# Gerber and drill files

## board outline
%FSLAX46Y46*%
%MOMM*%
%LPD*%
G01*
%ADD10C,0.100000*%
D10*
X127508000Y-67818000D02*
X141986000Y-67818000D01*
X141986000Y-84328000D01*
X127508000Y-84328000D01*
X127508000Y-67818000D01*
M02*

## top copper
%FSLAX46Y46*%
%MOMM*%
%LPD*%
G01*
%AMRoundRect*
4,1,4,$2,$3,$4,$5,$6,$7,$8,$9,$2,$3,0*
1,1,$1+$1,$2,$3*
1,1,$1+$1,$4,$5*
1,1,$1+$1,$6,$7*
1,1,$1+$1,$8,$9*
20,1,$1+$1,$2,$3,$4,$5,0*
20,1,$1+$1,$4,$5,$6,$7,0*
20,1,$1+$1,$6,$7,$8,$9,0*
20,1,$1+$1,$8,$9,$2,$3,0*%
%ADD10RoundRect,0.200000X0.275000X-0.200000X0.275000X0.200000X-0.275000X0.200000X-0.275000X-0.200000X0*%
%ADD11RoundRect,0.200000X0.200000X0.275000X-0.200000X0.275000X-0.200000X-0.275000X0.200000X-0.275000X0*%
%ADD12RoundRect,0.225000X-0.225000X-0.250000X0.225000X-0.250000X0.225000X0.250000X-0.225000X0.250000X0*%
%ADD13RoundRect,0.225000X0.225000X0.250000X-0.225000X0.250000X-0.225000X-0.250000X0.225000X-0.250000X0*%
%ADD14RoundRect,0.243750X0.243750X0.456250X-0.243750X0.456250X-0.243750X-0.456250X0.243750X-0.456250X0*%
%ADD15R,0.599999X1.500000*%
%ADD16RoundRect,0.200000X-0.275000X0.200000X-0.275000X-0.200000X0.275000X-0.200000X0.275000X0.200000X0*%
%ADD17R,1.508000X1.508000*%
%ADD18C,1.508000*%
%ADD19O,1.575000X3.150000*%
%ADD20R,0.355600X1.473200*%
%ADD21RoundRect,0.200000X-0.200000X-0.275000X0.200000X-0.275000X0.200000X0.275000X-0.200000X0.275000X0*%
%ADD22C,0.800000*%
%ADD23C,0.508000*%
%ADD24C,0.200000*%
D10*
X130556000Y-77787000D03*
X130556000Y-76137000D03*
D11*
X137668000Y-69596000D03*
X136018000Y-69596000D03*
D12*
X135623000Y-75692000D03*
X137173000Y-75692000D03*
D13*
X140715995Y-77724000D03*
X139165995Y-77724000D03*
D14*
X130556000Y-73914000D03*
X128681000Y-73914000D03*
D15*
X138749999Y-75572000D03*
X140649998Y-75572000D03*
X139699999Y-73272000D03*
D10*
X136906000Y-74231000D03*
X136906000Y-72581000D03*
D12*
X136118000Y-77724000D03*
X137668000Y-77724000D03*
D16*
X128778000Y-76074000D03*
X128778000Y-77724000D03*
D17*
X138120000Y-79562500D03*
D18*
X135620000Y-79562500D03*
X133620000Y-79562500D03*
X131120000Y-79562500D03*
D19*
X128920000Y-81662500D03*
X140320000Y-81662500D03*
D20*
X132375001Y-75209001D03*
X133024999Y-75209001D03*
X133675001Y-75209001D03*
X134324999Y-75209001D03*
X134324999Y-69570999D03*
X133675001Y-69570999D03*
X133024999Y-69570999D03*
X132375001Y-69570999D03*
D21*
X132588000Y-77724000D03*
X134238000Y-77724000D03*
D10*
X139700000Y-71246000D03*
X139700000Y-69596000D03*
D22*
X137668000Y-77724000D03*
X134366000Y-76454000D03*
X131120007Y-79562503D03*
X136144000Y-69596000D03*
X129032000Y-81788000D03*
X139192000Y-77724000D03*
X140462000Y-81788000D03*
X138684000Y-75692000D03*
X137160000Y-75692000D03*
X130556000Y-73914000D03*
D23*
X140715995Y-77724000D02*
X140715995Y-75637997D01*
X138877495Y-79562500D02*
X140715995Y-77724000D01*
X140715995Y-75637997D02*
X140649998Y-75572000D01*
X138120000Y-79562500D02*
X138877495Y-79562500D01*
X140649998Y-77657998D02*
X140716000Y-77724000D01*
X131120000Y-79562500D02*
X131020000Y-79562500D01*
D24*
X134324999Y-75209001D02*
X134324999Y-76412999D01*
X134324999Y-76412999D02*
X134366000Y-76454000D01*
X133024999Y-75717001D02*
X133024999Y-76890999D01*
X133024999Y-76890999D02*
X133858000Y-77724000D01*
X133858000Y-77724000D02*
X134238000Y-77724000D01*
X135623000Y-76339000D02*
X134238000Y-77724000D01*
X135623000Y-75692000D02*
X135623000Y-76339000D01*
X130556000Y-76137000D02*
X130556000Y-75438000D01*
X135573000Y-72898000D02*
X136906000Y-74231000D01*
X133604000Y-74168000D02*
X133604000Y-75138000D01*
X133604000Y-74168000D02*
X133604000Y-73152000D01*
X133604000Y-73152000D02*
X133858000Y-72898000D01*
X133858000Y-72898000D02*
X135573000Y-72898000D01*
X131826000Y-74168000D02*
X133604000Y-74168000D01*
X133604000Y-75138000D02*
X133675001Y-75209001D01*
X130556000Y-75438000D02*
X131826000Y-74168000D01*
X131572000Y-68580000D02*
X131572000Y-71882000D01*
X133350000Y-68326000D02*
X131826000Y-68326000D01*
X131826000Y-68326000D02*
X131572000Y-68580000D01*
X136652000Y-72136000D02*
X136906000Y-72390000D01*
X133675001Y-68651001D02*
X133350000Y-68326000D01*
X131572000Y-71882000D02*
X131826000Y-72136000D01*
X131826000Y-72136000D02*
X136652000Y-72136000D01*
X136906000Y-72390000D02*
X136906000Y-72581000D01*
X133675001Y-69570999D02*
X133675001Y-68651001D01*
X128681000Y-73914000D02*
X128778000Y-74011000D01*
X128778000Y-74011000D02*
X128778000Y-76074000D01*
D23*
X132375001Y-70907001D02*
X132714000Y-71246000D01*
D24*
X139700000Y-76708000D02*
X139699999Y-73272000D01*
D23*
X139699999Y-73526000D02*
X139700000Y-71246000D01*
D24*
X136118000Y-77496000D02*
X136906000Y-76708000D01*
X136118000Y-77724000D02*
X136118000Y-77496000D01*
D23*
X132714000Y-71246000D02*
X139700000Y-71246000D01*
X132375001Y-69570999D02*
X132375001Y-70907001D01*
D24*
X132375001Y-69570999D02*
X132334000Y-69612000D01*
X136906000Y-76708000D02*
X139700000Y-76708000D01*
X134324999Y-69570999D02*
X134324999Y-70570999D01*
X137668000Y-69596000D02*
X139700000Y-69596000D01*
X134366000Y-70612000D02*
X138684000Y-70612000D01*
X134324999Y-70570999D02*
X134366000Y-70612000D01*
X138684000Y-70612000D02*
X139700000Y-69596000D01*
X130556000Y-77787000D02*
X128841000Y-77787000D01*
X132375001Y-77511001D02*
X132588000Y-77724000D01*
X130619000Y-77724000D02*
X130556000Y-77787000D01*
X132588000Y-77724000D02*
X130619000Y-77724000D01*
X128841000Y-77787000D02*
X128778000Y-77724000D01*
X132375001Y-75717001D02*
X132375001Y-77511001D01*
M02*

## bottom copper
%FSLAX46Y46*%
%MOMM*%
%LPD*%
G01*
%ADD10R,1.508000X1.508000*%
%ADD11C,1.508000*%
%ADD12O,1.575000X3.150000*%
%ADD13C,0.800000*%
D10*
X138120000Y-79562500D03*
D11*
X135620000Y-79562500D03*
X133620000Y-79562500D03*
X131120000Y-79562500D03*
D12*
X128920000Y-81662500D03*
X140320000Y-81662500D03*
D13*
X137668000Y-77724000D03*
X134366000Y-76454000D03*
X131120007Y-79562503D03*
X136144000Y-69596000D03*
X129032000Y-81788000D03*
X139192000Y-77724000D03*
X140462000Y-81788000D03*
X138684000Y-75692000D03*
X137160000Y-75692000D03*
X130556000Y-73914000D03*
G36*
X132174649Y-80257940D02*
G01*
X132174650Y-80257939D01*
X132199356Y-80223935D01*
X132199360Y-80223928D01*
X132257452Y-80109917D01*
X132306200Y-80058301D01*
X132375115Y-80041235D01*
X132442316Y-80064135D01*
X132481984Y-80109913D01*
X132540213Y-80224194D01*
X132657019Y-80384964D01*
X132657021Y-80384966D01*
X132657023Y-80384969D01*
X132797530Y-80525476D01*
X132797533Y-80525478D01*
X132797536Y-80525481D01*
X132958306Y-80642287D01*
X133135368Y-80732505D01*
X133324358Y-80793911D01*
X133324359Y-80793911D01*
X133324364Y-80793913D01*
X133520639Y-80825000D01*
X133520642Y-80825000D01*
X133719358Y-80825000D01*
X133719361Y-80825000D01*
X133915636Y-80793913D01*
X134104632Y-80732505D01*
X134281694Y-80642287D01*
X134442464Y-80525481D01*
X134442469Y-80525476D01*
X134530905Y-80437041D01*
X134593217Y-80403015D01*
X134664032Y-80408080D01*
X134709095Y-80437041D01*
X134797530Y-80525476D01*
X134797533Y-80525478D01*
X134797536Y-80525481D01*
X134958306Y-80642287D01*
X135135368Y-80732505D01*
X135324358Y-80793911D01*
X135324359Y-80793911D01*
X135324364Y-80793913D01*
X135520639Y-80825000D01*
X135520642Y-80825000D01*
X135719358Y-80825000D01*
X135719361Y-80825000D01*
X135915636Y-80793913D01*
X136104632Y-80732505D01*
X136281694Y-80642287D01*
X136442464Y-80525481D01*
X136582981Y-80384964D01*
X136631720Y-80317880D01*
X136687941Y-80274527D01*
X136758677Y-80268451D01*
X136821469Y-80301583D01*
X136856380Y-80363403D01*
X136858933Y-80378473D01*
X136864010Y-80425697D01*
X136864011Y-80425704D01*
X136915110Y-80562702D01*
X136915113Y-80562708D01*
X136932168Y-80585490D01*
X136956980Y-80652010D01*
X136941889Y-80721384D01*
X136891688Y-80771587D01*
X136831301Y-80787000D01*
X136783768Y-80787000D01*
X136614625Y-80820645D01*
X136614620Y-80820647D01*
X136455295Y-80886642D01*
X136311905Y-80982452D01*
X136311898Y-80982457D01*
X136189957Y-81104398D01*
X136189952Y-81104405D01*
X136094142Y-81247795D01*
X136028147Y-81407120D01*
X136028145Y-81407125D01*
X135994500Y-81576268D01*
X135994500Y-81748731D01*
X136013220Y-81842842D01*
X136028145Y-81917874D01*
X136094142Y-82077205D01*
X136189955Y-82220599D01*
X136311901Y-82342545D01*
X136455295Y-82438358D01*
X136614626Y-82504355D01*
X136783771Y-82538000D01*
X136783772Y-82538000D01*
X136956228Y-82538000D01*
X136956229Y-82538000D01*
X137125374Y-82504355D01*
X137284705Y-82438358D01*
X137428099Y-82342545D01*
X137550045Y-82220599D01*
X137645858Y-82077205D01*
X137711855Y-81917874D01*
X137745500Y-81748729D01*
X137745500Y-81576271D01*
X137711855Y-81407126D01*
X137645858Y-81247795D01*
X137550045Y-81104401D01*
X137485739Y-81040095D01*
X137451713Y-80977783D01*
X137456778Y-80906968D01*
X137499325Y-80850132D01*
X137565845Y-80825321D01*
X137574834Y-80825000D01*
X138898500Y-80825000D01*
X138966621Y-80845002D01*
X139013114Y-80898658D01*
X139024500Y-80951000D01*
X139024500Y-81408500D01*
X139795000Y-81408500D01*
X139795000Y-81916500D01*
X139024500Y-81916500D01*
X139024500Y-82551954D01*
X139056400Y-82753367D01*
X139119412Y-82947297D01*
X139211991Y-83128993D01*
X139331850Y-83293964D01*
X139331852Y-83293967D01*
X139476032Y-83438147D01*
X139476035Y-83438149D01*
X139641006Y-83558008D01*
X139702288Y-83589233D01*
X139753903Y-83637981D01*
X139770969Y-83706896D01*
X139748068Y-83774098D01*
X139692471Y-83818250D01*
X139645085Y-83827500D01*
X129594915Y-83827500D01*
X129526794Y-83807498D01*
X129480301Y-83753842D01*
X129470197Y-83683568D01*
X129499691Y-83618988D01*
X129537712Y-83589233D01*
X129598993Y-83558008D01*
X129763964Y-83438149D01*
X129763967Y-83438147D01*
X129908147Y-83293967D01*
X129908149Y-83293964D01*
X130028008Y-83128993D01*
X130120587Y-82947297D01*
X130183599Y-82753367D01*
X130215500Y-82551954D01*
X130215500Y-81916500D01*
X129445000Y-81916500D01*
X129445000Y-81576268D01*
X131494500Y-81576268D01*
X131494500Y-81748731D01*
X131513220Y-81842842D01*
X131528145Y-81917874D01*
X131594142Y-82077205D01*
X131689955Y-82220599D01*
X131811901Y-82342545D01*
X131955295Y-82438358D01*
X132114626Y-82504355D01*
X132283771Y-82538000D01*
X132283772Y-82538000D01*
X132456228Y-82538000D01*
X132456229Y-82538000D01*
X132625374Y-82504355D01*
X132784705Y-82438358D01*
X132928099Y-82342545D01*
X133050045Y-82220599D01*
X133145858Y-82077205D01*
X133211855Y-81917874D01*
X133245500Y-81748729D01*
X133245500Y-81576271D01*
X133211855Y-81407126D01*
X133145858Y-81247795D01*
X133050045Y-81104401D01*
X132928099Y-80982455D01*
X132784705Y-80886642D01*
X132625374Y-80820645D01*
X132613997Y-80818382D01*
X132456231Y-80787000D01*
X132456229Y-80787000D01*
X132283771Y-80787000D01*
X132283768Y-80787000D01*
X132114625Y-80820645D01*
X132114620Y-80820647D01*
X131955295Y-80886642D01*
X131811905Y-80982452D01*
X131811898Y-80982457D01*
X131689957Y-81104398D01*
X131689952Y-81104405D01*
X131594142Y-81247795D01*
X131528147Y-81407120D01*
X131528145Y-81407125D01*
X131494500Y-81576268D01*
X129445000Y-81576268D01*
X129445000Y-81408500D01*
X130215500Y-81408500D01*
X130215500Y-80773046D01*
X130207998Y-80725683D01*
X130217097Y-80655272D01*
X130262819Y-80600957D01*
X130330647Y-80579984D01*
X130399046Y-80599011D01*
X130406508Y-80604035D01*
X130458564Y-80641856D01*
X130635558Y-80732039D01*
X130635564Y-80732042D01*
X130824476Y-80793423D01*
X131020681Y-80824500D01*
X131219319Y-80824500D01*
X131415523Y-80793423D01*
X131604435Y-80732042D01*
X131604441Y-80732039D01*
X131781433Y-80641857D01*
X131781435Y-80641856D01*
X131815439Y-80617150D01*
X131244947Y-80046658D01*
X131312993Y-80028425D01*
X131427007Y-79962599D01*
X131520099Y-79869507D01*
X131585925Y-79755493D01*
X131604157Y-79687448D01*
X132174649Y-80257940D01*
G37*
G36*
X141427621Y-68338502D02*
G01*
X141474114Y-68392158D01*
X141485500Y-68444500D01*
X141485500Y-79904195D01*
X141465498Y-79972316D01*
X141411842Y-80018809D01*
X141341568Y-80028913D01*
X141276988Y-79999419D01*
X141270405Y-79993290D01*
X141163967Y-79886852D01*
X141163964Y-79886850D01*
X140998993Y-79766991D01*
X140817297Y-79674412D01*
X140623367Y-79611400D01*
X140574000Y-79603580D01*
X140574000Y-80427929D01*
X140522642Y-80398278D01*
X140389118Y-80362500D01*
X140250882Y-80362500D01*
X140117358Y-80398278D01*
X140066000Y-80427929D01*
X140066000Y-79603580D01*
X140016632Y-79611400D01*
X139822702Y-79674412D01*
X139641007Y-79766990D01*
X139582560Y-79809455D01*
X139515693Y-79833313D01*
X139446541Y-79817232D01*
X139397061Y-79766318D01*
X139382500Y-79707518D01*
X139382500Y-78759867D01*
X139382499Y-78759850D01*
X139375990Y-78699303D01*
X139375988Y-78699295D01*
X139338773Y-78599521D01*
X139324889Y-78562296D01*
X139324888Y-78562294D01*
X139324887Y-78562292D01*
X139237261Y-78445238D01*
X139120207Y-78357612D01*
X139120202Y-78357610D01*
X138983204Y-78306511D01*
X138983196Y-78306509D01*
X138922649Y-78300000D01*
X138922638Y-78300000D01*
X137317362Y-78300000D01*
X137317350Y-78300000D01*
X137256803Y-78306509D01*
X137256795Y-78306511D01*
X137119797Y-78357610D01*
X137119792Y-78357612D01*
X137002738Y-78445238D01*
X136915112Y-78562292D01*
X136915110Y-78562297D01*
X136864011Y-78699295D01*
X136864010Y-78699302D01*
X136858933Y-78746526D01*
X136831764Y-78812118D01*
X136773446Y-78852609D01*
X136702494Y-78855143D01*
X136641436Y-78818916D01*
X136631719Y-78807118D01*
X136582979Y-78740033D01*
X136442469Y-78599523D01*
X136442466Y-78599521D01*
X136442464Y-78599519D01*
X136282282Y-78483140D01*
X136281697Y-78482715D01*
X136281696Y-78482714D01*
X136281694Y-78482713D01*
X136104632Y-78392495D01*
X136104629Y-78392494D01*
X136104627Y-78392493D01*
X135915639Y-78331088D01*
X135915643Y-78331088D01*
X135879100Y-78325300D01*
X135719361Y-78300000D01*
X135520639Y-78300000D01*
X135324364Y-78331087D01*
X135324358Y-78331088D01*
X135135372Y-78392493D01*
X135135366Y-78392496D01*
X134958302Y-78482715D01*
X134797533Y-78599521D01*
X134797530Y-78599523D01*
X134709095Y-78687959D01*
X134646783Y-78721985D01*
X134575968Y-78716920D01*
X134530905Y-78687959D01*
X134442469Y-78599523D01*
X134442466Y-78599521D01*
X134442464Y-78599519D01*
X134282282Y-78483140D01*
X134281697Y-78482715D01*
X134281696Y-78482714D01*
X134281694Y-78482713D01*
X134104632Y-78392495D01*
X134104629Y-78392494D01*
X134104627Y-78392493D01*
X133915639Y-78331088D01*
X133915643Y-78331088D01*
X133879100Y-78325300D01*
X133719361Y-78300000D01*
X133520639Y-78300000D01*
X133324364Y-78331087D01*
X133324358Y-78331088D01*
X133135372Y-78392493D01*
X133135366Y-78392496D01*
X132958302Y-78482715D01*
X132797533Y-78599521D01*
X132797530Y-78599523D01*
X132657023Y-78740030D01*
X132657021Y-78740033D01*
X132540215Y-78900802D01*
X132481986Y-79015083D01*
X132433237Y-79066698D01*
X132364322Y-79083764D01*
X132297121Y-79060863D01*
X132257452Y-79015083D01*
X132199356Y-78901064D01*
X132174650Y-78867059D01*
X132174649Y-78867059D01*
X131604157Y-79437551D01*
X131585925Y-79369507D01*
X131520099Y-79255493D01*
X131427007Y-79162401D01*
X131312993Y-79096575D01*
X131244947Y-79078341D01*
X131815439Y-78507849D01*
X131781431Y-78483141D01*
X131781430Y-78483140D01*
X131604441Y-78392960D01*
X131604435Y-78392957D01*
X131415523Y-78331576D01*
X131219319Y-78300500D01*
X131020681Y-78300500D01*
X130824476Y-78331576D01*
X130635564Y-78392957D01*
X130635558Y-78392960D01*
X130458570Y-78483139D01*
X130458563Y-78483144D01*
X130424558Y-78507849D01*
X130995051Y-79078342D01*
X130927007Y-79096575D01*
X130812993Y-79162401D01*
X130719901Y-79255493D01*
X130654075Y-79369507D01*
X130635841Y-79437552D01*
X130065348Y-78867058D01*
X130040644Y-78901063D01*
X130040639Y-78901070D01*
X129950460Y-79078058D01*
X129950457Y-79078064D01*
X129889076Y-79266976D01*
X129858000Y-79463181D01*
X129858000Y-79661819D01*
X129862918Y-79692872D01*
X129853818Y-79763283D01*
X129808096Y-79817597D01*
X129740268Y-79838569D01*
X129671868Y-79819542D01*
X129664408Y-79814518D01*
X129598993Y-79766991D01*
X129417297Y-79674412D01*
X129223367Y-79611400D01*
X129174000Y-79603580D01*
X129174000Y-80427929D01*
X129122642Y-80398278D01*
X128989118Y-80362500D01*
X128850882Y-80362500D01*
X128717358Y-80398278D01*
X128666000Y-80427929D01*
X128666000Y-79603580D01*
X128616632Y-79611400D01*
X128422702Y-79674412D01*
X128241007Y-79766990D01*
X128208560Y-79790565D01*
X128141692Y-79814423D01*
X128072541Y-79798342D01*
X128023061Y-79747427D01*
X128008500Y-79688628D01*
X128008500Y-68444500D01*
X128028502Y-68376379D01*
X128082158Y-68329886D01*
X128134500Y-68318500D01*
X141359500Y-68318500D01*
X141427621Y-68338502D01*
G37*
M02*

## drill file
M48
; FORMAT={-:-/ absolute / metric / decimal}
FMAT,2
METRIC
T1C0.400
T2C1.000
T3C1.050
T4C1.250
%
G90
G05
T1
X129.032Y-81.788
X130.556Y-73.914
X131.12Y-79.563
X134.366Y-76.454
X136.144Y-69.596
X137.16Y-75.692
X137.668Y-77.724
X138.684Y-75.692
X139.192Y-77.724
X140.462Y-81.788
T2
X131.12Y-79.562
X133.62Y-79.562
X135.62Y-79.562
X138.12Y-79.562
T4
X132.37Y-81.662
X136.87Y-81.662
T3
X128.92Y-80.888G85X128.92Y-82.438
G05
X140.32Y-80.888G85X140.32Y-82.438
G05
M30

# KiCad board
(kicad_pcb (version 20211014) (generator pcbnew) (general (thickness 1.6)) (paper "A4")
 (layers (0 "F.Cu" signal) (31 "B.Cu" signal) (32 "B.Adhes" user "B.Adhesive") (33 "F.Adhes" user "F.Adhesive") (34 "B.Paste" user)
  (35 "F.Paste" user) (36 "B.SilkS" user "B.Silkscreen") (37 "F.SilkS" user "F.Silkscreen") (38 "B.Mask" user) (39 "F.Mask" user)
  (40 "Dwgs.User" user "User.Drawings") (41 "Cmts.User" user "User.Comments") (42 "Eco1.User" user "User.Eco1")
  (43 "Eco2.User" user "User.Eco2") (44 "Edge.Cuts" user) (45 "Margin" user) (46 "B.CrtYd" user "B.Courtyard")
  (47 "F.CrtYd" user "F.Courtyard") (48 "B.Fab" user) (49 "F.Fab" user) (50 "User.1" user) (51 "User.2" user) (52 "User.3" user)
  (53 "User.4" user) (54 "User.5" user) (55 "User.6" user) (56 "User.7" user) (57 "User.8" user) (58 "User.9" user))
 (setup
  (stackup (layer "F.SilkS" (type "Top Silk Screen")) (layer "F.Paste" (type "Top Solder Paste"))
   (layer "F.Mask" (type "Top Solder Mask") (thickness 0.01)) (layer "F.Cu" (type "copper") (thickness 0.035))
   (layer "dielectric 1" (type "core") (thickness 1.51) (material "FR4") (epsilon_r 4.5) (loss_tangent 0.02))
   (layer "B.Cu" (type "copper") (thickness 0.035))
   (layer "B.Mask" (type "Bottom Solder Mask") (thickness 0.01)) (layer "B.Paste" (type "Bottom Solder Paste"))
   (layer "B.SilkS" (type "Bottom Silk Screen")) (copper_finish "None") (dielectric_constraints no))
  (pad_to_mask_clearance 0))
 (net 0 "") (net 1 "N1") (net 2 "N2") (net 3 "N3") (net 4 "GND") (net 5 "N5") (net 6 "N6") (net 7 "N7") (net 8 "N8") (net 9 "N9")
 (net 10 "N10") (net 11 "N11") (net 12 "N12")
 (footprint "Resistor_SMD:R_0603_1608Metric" (layer "F.Cu") (at 130.556 76.962 90)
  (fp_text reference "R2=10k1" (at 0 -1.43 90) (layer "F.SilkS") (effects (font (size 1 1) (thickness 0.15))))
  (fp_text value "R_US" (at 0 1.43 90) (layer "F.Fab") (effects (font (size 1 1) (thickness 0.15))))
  (pad "1" smd roundrect (at -0.825 0 90) (size 0.8 0.95) (layers "F.Cu" "F.Paste" "F.Mask") (roundrect_rratio 0.25) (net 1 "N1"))
  (pad "2" smd roundrect (at 0.825 0 90) (size 0.8 0.95) (layers "F.Cu" "F.Paste" "F.Mask") (roundrect_rratio 0.25) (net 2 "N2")))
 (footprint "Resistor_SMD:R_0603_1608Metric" (layer "F.Cu") (at 136.843 69.596 180)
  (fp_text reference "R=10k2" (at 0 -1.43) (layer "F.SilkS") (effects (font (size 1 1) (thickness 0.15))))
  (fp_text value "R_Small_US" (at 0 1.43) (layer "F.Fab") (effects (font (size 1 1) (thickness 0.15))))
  (pad "1" smd roundrect (at -0.825 0 180) (size 0.8 0.95) (layers "F.Cu" "F.Paste" "F.Mask") (roundrect_rratio 0.25) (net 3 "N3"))
  (pad "2" smd roundrect (at 0.825 0 180) (size 0.8 0.95) (layers "F.Cu" "F.Paste" "F.Mask") (roundrect_rratio 0.25) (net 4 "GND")))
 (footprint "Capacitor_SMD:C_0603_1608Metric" (layer "F.Cu") (at 136.398 75.692)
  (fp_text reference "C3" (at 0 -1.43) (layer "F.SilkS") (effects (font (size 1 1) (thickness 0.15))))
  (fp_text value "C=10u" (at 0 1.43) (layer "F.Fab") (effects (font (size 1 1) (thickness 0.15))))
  (pad "1" smd roundrect (at -0.775 0) (size 0.9 0.95) (layers "F.Cu" "F.Paste" "F.Mask") (roundrect_rratio 0.25) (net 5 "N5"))
  (pad "2" smd roundrect (at 0.775 0) (size 0.9 0.95) (layers "F.Cu" "F.Paste" "F.Mask") (roundrect_rratio 0.25) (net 4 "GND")))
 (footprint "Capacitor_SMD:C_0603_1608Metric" (layer "F.Cu") (at 139.940995 77.724 180)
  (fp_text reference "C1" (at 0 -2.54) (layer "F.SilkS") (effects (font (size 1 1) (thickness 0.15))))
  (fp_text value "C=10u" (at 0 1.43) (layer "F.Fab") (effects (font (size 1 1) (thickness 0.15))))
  (pad "1" smd roundrect (at -0.775 0 180) (size 0.9 0.95) (layers "F.Cu" "F.Paste" "F.Mask") (roundrect_rratio 0.25) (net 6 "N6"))
  (pad "2" smd roundrect (at 0.775 0 180) (size 0.9 0.95) (layers "F.Cu" "F.Paste" "F.Mask") (roundrect_rratio 0.25) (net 4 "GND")))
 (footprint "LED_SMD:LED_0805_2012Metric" (layer "F.Cu") (at 129.6185 73.914 180)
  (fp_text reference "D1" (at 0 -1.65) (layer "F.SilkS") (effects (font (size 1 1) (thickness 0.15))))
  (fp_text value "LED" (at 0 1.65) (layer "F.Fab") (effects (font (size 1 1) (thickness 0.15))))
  (pad "1" smd roundrect (at -0.9375 0 180) (size 0.975 1.4) (layers "F.Cu" "F.Paste" "F.Mask") (roundrect_rratio 0.25) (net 4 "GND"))
  (pad "2" smd roundrect (at 0.9375 0 180) (size 0.975 1.4) (layers "F.Cu" "F.Paste" "F.Mask") (roundrect_rratio 0.25) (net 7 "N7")))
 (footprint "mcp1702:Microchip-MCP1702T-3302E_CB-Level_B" (layer "F.Cu") (at 139.7 74.422 90)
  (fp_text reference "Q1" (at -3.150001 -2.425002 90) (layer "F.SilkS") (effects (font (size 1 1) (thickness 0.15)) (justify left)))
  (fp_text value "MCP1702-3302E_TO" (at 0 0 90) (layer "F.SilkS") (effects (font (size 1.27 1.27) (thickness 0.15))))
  (pad "1" smd rect locked (at -1.15 -0.950001) (size 0.599999 1.5) (layers "F.Cu" "F.Paste" "F.Mask") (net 4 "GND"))
  (pad "2" smd rect locked (at -1.15 0.949998) (size 0.599999 1.5) (layers "F.Cu" "F.Paste" "F.Mask") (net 6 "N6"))
  (pad "3" smd rect locked (at 1.15 -0.000001) (size 0.599999 1.5) (layers "F.Cu" "F.Paste" "F.Mask") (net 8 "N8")))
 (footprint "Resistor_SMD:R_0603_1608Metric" (layer "F.Cu") (at 136.906 73.406 90)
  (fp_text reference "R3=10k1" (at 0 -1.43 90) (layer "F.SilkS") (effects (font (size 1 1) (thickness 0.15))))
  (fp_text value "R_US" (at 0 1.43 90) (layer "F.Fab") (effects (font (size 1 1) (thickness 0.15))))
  (pad "1" smd roundrect (at -0.825 0 90) (size 0.8 0.95) (layers "F.Cu" "F.Paste" "F.Mask") (roundrect_rratio 0.25) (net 2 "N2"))
  (pad "2" smd roundrect (at 0.825 0 90) (size 0.8 0.95) (layers "F.Cu" "F.Paste" "F.Mask") (roundrect_rratio 0.25) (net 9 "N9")))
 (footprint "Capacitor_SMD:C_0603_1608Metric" (layer "F.Cu") (at 136.893 77.724)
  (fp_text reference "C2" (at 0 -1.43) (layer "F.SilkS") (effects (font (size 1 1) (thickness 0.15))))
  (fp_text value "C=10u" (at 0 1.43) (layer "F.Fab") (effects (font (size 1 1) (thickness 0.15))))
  (pad "1" smd roundrect (at -0.775 0) (size 0.9 0.95) (layers "F.Cu" "F.Paste" "F.Mask") (roundrect_rratio 0.25) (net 8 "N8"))
  (pad "2" smd roundrect (at 0.775 0) (size 0.9 0.95) (layers "F.Cu" "F.Paste" "F.Mask") (roundrect_rratio 0.25) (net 4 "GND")))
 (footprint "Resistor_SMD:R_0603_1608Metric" (layer "F.Cu") (at 128.778 76.899 -90)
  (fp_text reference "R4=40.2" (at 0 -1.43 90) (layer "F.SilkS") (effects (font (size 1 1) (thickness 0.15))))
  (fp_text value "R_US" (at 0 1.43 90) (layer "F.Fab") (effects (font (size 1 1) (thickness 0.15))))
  (pad "1" smd roundrect (at -0.825 0 270) (size 0.8 0.95) (layers "F.Cu" "F.Paste" "F.Mask") (roundrect_rratio 0.25) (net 7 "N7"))
  (pad "2" smd roundrect (at 0.825 0 270) (size 0.8 0.95) (layers "F.Cu" "F.Paste" "F.Mask") (roundrect_rratio 0.25) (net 1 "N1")))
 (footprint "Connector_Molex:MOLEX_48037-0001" (layer "F.Cu") (at 134.62 81.6625)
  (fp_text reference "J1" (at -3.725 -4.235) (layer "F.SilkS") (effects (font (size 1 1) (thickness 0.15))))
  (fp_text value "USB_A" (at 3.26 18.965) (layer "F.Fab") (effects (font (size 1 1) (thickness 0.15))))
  (pad "" np_thru_hole circle (at -2.25 0) (size 1.25 1.25) (drill 1.25) (layers *.Cu *.Mask))
  (pad "" np_thru_hole circle (at 2.25 0) (size 1.25 1.25) (drill 1.25) (layers *.Cu *.Mask))
  (pad "1" thru_hole rect (at 3.5 -2.1) (size 1.508 1.508) (drill 1) (layers *.Cu *.Mask) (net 6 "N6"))
  (pad "2" thru_hole circle (at 1 -2.1) (size 1.508 1.508) (drill 1) (layers *.Cu *.Mask) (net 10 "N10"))
  (pad "3" thru_hole circle (at -1 -2.1) (size 1.508 1.508) (drill 1) (layers *.Cu *.Mask) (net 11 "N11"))
  (pad "4" thru_hole circle (at -3.5 -2.1) (size 1.508 1.508) (drill 1) (layers *.Cu *.Mask) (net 4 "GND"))
  (pad "5" thru_hole oval (at -5.7 0) (size 1.575 3.15) (drill oval 1.05 2.6) (layers *.Cu *.Mask) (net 4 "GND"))
  (pad "5" thru_hole oval (at 5.7 0) (size 1.575 3.15) (drill oval 1.05 2.6) (layers *.Cu *.Mask) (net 4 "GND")))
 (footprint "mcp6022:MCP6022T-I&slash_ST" (layer "F.Cu") (at 133.35 72.39 90)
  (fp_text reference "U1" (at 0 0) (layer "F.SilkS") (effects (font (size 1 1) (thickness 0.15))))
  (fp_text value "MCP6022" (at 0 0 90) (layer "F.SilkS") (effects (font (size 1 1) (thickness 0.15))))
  (pad "1" smd rect locked (at -2.819001 -0.974999 90) (size 1.4732 0.3556) (layers "F.Cu" "F.Paste" "F.Mask") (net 1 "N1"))
  (pad "2" smd rect locked (at -2.819001 -0.325001 90) (size 1.4732 0.3556) (layers "F.Cu" "F.Paste" "F.Mask") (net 5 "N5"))
  (pad "3" smd rect locked (at -2.819001 0.325001 90) (size 1.4732 0.3556) (layers "F.Cu" "F.Paste" "F.Mask") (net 2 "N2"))
  (pad "4" smd rect locked (at -2.819001 0.974999 90) (size 1.4732 0.3556) (layers "F.Cu" "F.Paste" "F.Mask") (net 4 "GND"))
  (pad "5" smd rect locked (at 2.819001 0.974999 90) (size 1.4732 0.3556) (layers "F.Cu" "F.Paste" "F.Mask") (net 3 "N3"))
  (pad "6" smd rect locked (at 2.819001 0.325001 90) (size 1.4732 0.3556) (layers "F.Cu" "F.Paste" "F.Mask") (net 9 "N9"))
  (pad "7" smd rect locked (at 2.819001 -0.325001 90) (size 1.4732 0.3556) (layers "F.Cu" "F.Paste" "F.Mask") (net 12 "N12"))
  (pad "8" smd rect locked (at 2.819001 -0.974999 90) (size 1.4732 0.3556) (layers "F.Cu" "F.Paste" "F.Mask") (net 8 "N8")))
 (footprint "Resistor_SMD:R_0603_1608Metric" (layer "F.Cu") (at 133.413 77.724)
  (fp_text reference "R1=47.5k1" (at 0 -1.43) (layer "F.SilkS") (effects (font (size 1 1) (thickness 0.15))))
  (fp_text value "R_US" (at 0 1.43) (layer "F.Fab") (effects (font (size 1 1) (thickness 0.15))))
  (pad "1" smd roundrect (at -0.825 0) (size 0.8 0.95) (layers "F.Cu" "F.Paste" "F.Mask") (roundrect_rratio 0.25) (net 1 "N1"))
  (pad "2" smd roundrect (at 0.825 0) (size 0.8 0.95) (layers "F.Cu" "F.Paste" "F.Mask") (roundrect_rratio 0.25) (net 5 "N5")))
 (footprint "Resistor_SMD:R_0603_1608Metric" (layer "F.Cu") (at 139.7 70.421 90)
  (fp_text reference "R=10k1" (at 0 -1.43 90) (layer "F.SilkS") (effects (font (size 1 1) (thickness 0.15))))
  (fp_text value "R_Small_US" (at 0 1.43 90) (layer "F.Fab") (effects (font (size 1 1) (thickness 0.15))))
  (pad "1" smd roundrect (at -0.825 0 90) (size 0.8 0.95) (layers "F.Cu" "F.Paste" "F.Mask") (roundrect_rratio 0.25) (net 8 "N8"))
  (pad "2" smd roundrect (at 0.825 0 90) (size 0.8 0.95) (layers "F.Cu" "F.Paste" "F.Mask") (roundrect_rratio 0.25) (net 3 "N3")))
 (gr_rect (start 127.508 67.818) (end 141.986 84.328) (layer "Edge.Cuts") (width 0.1) (fill none))
 (segment (start 140.715995 77.724) (end 140.715995 75.637997) (width 0.508) (layer "F.Cu") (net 6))
 (segment (start 138.877495 79.5625) (end 140.715995 77.724) (width 0.508) (layer "F.Cu") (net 6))
 (segment (start 140.715995 75.637997) (end 140.649998 75.572) (width 0.508) (layer "F.Cu") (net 6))
 (segment (start 138.12 79.5625) (end 138.877495 79.5625) (width 0.508) (layer "F.Cu") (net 6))
 (segment (start 140.649998 77.657998) (end 140.716 77.724) (width 0.508) (layer "F.Cu") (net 6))
 (segment (start 131.12 79.5625) (end 131.02 79.5625) (width 0.508) (layer "F.Cu") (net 4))
 (segment (start 134.324999 75.209001) (end 134.324999 76.412999) (width 0.2) (layer "F.Cu") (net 4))
 (segment (start 134.324999 76.412999) (end 134.366 76.454) (width 0.2) (layer "F.Cu") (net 4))
 (via (at 137.668 77.724) (size 0.8) (drill 0.4) (layers "F.Cu" "B.Cu") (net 4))
 (via (at 134.366 76.454) (size 0.8) (drill 0.4) (layers "F.Cu" "B.Cu") (free) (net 4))
 (via (at 131.120007 79.562503) (size 0.8) (drill 0.4) (layers "F.Cu" "B.Cu") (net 4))
 (via (at 136.144 69.596) (size 0.8) (drill 0.4) (layers "F.Cu" "B.Cu") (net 4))
 (via (at 129.032 81.788) (size 0.8) (drill 0.4) (layers "F.Cu" "B.Cu") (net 4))
 (via (at 139.192 77.724) (size 0.8) (drill 0.4) (layers "F.Cu" "B.Cu") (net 4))
 (via (at 140.462 81.788) (size 0.8) (drill 0.4) (layers "F.Cu" "B.Cu") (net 4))
 (via (at 138.684 75.692) (size 0.8) (drill 0.4) (layers "F.Cu" "B.Cu") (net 4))
 (via (at 137.16 75.692) (size 0.8) (drill 0.4) (layers "F.Cu" "B.Cu") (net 4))
 (via (at 130.556 73.914) (size 0.8) (drill 0.4) (layers "F.Cu" "B.Cu") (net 4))
 (segment (start 133.024999 75.717001) (end 133.024999 76.890999) (width 0.2) (layer "F.Cu") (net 5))
 (segment (start 133.024999 76.890999) (end 133.858 77.724) (width 0.2) (layer "F.Cu") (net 5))
 (segment (start 133.858 77.724) (end 134.238 77.724) (width 0.2) (layer "F.Cu") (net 5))
 (segment (start 135.623 76.339) (end 134.238 77.724) (width 0.2) (layer "F.Cu") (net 5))
 (segment (start 135.623 75.692) (end 135.623 76.339) (width 0.2) (layer "F.Cu") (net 5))
 (segment (start 130.556 76.137) (end 130.556 75.438) (width 0.2) (layer "F.Cu") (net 2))
 (segment (start 135.573 72.898) (end 136.906 74.231) (width 0.2) (layer "F.Cu") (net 2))
 (segment (start 133.604 74.168) (end 133.604 75.138) (width 0.2) (layer "F.Cu") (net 2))
 (segment (start 133.604 74.168) (end 133.604 73.152) (width 0.2) (layer "F.Cu") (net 2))
 (segment (start 133.604 73.152) (end 133.858 72.898) (width 0.2) (layer "F.Cu") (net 2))
 (segment (start 133.858 72.898) (end 135.573 72.898) (width 0.2) (layer "F.Cu") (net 2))
 (segment (start 131.826 74.168) (end 133.604 74.168) (width 0.2) (layer "F.Cu") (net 2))
 (segment (start 133.604 75.138) (end 133.675001 75.209001) (width 0.2) (layer "F.Cu") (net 2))
 (segment (start 130.556 75.438) (end 131.826 74.168) (width 0.2) (layer "F.Cu") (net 2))
 (segment (start 131.572 68.58) (end 131.572 71.882) (width 0.2) (layer "F.Cu") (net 9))
 (segment (start 133.35 68.326) (end 131.826 68.326) (width 0.2) (layer "F.Cu") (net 9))
 (segment (start 131.826 68.326) (end 131.572 68.58) (width 0.2) (layer "F.Cu") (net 9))
 (segment (start 136.652 72.136) (end 136.906 72.39) (width 0.2) (layer "F.Cu") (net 9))
 (segment (start 133.675001 68.651001) (end 133.35 68.326) (width 0.2) (layer "F.Cu") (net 9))
 (segment (start 131.572 71.882) (end 131.826 72.136) (width 0.2) (layer "F.Cu") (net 9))
 (segment (start 131.826 72.136) (end 136.652 72.136) (width 0.2) (layer "F.Cu") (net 9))
 (segment (start 136.906 72.39) (end 136.906 72.581) (width 0.2) (layer "F.Cu") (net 9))
 (segment (start 133.675001 69.570999) (end 133.675001 68.651001) (width 0.2) (layer "F.Cu") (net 9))
 (segment (start 128.681 73.914) (end 128.778 74.011) (width 0.2) (layer "F.Cu") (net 7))
 (segment (start 128.778 74.011) (end 128.778 76.074) (width 0.2) (layer "F.Cu") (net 7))
 (segment (start 132.375001 70.907001) (end 132.714 71.246) (width 0.508) (layer "F.Cu") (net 8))
 (segment (start 139.7 76.708) (end 139.699999 73.272) (width 0.2) (layer "F.Cu") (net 8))
 (segment (start 139.699999 73.526) (end 139.7 71.246) (width 0.508) (layer "F.Cu") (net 8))
 (segment (start 136.118 77.496) (end 136.906 76.708) (width 0.2) (layer "F.Cu") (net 8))
 (segment (start 136.118 77.724) (end 136.118 77.496) (width 0.2) (layer "F.Cu") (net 8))
 (segment (start 132.714 71.246) (end 139.7 71.246) (width 0.508) (layer "F.Cu") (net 8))
 (segment (start 132.375001 69.570999) (end 132.375001 70.907001) (width 0.508) (layer "F.Cu") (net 8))
 (segment (start 132.375001 69.570999) (end 132.334 69.612) (width 0.2) (layer "F.Cu") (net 8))
 (segment (start 136.906 76.708) (end 139.7 76.708) (width 0.2) (layer "F.Cu") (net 8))
 (segment (start 134.324999 69.570999) (end 134.324999 70.570999) (width 0.2) (layer "F.Cu") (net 3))
 (segment (start 137.668 69.596) (end 139.7 69.596) (width 0.2) (layer "F.Cu") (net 3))
 (segment (start 134.366 70.612) (end 138.684 70.612) (width 0.2) (layer "F.Cu") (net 3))
 (segment (start 134.324999 70.570999) (end 134.366 70.612) (width 0.2) (layer "F.Cu") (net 3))
 (segment (start 138.684 70.612) (end 139.7 69.596) (width 0.2) (layer "F.Cu") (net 3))
 (segment (start 130.556 77.787) (end 128.841 77.787) (width 0.2) (layer "F.Cu") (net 1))
 (segment (start 132.375001 77.511001) (end 132.588 77.724) (width 0.2) (layer "F.Cu") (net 1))
 (segment (start 130.619 77.724) (end 130.556 77.787) (width 0.2) (layer "F.Cu") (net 1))
 (segment (start 132.588 77.724) (end 130.619 77.724) (width 0.2) (layer "F.Cu") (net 1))
 (segment (start 128.841 77.787) (end 128.778 77.724) (width 0.2) (layer "F.Cu") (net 1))
 (segment (start 132.375001 75.717001) (end 132.375001 77.511001) (width 0.2) (layer "F.Cu") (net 1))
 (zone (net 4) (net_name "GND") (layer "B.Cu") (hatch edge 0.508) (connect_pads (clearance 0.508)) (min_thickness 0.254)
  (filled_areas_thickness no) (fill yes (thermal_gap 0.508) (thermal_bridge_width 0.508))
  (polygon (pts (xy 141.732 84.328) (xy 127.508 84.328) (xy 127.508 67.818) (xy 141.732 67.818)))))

